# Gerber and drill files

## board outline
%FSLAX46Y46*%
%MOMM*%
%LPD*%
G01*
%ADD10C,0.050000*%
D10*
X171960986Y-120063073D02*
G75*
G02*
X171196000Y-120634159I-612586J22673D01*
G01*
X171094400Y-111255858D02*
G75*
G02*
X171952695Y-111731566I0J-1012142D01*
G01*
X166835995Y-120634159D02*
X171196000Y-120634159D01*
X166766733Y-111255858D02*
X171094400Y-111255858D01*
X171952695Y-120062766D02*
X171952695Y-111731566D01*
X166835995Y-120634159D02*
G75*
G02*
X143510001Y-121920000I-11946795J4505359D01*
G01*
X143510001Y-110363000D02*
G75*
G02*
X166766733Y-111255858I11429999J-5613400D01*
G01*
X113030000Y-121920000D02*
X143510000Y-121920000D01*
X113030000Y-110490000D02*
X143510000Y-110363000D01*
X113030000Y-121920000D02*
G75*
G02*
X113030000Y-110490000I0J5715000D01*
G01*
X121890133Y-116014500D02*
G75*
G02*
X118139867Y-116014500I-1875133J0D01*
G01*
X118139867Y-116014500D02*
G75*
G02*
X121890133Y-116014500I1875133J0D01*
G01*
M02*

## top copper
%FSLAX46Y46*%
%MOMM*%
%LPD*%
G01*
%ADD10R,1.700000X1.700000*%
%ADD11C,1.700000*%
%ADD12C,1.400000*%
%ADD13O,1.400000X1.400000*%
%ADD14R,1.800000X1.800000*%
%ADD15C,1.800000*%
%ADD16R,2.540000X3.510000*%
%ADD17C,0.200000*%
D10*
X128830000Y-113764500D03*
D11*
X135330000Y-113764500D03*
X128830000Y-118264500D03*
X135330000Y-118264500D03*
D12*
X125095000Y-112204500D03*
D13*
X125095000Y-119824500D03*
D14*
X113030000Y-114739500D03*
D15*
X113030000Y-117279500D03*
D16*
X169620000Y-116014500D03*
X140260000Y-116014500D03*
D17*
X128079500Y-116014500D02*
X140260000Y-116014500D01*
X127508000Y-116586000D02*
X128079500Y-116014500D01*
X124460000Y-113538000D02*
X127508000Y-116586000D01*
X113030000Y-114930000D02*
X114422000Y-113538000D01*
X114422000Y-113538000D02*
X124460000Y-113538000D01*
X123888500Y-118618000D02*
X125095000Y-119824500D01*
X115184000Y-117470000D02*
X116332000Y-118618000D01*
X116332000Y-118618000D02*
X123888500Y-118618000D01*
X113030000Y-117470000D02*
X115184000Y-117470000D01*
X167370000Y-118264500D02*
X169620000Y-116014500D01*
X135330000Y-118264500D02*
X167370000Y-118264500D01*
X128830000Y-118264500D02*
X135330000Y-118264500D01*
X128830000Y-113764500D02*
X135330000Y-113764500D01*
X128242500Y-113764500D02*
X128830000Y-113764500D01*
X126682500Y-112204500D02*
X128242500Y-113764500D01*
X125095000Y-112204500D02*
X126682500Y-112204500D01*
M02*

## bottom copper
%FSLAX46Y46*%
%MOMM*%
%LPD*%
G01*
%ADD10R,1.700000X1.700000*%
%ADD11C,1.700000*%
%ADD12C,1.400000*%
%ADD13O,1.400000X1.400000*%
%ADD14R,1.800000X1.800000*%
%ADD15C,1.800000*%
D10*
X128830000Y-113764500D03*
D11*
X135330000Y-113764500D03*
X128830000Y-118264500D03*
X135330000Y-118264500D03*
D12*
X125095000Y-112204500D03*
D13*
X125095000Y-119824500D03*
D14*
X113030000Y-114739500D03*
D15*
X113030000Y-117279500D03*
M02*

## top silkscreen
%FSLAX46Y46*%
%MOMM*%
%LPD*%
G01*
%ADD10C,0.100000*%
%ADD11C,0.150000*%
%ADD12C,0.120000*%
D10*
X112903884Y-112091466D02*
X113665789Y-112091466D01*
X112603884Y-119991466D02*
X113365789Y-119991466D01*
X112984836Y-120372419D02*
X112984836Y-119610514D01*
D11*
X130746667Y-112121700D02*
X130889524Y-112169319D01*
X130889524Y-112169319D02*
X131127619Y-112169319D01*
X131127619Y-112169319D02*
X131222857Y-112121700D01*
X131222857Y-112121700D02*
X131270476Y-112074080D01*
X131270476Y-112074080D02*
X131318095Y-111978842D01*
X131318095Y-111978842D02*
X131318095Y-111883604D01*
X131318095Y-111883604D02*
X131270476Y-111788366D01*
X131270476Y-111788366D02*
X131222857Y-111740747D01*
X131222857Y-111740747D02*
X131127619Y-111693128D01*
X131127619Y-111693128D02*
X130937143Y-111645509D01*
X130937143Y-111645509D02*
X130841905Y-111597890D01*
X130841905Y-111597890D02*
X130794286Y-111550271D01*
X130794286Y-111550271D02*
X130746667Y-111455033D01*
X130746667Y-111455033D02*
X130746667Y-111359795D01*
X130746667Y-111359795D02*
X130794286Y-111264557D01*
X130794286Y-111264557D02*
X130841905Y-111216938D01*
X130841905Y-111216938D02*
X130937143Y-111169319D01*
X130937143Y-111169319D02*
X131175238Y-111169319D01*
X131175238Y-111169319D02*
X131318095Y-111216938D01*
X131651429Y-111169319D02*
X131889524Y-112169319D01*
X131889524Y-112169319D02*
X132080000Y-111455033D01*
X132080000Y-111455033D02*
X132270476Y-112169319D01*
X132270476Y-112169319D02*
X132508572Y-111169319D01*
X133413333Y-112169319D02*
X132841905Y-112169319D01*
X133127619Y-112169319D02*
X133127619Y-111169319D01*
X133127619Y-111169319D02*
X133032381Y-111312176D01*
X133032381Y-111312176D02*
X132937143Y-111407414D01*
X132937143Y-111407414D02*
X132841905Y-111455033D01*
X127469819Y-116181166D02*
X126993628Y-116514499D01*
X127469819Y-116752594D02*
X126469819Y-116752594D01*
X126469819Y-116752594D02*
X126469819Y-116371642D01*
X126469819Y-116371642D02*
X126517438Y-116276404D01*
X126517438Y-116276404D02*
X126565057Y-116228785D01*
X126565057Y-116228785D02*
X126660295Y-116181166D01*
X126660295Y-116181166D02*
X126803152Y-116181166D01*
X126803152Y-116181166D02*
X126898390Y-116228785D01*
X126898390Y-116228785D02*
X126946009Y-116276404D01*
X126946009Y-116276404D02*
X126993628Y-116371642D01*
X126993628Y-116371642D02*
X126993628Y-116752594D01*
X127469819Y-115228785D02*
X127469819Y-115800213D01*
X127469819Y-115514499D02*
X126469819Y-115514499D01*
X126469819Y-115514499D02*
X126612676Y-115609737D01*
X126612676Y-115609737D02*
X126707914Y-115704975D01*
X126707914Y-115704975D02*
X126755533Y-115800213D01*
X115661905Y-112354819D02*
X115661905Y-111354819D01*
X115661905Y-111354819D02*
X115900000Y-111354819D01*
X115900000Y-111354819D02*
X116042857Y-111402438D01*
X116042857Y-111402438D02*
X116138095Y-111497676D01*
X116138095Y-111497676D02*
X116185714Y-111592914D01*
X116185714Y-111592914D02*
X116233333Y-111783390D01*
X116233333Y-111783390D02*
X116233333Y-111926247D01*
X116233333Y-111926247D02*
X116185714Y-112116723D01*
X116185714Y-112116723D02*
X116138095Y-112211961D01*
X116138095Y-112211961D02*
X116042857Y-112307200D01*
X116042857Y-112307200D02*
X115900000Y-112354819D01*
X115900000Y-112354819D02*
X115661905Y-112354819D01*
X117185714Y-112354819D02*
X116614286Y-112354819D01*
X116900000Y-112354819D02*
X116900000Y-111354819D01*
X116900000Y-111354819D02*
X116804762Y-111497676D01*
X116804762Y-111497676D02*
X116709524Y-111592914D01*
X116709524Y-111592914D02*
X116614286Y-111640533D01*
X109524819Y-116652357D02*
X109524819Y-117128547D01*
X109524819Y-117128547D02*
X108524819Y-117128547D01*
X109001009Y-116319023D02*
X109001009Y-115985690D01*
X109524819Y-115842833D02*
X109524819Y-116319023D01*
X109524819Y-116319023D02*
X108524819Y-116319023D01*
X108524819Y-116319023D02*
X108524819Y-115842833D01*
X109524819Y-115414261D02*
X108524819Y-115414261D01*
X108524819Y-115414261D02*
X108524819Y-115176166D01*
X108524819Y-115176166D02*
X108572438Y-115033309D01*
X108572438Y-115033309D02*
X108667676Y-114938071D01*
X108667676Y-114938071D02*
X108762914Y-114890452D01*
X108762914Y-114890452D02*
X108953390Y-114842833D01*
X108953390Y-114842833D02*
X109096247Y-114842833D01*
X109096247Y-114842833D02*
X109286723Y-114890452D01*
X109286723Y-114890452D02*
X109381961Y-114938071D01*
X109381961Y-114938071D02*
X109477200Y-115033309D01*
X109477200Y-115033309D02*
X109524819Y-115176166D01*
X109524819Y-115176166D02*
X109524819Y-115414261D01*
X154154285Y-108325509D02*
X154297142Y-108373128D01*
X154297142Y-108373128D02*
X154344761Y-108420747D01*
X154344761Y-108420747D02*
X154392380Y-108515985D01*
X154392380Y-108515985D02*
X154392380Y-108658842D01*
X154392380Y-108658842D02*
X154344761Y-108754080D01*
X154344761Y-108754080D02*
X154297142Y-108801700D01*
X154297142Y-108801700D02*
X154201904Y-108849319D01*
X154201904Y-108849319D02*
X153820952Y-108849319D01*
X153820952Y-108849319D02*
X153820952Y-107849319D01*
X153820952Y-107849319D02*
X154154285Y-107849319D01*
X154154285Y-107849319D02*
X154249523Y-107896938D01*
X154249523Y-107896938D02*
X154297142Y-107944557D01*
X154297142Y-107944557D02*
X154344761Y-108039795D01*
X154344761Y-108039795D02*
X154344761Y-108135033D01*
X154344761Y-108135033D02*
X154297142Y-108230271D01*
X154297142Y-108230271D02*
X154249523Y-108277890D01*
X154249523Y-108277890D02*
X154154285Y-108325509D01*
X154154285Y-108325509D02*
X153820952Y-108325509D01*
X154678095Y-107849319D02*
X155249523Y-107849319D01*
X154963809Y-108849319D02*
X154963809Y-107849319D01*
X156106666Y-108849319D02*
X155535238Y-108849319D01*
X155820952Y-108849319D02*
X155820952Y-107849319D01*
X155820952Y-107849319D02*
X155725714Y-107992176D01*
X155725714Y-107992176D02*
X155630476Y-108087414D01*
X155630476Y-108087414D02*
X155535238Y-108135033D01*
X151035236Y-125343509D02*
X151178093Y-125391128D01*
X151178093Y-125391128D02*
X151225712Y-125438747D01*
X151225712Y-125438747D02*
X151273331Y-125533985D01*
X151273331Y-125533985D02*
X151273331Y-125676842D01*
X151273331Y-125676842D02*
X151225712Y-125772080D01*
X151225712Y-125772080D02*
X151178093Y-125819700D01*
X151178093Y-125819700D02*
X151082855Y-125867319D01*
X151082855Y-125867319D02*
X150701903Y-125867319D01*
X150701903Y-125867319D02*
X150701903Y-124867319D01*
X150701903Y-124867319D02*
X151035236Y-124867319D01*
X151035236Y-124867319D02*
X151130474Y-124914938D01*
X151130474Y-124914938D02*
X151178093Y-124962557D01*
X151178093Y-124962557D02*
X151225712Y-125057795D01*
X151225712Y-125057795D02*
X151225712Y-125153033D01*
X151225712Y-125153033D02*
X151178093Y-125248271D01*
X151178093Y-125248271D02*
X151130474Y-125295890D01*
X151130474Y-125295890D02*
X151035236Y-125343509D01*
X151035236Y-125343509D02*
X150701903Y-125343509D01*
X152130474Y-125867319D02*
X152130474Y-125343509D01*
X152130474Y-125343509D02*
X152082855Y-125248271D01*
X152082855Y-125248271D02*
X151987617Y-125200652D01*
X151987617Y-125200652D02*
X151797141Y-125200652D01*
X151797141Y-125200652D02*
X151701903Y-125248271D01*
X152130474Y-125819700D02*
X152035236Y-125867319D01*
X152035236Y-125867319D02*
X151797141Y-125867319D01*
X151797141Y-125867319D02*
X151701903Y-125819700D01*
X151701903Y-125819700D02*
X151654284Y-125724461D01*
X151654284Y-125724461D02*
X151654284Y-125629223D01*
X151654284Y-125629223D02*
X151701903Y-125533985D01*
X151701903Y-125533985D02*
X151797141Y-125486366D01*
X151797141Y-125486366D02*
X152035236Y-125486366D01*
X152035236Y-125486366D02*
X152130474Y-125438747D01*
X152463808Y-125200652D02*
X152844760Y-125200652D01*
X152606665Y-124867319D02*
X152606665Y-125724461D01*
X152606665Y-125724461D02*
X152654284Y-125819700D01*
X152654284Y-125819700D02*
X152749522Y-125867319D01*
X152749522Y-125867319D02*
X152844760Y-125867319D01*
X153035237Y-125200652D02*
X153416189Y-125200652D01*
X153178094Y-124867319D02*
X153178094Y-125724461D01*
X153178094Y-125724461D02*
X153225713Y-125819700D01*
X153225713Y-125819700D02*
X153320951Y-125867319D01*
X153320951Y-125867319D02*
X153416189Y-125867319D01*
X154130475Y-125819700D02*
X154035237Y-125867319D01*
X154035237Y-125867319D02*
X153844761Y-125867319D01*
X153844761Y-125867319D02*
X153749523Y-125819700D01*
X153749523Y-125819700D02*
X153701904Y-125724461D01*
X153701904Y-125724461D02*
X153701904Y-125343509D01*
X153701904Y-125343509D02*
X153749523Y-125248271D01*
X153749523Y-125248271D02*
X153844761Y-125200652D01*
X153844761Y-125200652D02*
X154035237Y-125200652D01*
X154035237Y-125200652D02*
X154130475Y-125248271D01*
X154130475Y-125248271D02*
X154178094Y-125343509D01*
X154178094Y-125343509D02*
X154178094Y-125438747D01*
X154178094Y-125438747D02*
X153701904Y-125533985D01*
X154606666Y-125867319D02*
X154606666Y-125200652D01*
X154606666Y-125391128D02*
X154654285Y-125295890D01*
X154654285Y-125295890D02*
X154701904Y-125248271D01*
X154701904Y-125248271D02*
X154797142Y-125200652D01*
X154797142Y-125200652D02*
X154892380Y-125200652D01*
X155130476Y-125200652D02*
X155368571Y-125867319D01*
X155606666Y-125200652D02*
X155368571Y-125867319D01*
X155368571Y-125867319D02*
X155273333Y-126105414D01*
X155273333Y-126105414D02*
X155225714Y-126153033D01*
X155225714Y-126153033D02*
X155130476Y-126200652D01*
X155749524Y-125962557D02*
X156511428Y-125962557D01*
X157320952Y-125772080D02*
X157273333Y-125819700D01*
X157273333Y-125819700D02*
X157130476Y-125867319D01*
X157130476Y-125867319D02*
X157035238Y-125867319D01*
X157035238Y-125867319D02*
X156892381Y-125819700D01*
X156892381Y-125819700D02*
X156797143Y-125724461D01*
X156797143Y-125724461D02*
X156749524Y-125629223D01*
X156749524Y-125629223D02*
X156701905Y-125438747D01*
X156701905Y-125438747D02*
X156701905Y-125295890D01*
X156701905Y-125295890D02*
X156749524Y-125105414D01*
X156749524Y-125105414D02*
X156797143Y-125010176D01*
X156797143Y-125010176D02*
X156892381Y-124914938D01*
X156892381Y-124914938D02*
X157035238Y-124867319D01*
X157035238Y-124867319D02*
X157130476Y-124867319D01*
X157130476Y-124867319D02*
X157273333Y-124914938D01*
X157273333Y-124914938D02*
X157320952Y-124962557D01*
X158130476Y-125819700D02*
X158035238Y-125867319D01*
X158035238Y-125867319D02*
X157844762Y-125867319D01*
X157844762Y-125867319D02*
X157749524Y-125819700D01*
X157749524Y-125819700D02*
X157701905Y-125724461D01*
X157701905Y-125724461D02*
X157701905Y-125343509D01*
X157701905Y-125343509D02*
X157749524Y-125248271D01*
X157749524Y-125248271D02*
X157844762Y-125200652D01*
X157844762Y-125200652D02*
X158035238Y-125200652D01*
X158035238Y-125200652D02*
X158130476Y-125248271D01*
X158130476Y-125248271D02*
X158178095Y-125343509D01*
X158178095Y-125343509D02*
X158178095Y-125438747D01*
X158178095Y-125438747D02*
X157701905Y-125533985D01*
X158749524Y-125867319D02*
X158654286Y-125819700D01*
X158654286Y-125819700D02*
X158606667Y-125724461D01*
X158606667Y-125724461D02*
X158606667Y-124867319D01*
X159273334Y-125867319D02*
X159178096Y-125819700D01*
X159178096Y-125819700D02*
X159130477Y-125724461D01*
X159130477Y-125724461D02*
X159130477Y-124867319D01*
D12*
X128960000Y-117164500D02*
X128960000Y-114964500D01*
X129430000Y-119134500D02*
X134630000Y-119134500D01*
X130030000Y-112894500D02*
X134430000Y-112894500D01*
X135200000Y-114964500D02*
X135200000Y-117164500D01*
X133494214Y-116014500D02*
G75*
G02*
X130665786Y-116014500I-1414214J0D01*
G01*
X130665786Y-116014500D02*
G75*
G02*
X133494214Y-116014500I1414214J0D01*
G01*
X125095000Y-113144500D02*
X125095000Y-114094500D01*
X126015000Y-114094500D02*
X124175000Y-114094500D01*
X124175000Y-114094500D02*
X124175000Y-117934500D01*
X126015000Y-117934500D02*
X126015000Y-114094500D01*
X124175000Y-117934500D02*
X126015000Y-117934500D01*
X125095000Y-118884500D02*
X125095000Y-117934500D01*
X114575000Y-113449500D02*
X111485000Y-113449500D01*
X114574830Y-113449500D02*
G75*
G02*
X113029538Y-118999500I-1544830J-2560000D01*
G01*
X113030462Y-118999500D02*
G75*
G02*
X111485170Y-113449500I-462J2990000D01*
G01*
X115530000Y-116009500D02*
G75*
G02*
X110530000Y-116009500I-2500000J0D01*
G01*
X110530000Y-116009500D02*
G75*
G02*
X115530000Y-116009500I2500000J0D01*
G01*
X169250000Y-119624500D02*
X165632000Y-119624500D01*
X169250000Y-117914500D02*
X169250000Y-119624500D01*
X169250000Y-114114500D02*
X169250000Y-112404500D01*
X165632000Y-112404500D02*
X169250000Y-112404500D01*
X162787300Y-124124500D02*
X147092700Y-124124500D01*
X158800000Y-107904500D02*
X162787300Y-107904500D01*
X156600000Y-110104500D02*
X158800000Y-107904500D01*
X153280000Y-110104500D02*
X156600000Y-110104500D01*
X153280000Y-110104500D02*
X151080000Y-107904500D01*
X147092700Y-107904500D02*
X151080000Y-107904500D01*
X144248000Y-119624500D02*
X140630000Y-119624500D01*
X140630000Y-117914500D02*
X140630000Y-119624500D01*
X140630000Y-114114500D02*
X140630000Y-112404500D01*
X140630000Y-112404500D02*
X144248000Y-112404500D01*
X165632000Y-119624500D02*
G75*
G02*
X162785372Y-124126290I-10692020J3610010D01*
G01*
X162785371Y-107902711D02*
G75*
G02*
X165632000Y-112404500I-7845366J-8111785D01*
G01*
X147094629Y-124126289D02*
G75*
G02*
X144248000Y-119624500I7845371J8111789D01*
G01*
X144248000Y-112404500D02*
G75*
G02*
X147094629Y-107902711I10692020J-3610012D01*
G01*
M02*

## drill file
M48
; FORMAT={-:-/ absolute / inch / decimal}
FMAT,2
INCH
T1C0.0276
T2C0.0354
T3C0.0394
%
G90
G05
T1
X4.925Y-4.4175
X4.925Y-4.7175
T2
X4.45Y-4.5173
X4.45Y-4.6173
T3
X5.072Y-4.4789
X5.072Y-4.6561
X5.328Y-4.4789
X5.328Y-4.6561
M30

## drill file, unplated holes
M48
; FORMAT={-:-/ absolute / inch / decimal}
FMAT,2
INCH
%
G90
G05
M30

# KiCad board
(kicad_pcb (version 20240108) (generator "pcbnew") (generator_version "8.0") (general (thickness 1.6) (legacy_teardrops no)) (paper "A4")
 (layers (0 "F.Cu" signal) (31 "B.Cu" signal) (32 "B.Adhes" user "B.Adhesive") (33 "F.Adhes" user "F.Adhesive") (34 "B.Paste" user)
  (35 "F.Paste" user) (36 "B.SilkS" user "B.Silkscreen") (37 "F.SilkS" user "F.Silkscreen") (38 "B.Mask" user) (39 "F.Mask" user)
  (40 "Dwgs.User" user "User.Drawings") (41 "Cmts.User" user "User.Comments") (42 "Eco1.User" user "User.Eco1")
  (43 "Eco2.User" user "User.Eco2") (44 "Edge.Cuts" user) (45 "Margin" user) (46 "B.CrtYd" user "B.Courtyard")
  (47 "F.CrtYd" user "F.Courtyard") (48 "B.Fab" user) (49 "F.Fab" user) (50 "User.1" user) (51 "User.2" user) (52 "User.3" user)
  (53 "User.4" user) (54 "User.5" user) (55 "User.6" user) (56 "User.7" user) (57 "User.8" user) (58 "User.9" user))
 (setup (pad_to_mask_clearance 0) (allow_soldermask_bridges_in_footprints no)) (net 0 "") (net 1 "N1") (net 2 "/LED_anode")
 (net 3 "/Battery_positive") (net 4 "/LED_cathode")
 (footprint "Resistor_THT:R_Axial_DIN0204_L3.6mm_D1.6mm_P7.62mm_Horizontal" (layer "F.Cu") (at 125.095 112.2045 -90)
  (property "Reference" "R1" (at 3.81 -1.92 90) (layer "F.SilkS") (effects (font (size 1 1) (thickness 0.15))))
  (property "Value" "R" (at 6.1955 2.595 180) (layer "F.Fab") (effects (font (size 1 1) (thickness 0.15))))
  (fp_line (start 1.89 0.92) (end 5.73 0.92) (stroke (width 0.12) (type solid)) (layer "F.SilkS"))
  (fp_line (start 5.73 0.92) (end 5.73 -0.92) (stroke (width 0.12) (type solid)) (layer "F.SilkS"))
  (fp_line (start 0.94 0) (end 1.89 0) (stroke (width 0.12) (type solid)) (layer "F.SilkS"))
  (fp_line (start 6.68 0) (end 5.73 0) (stroke (width 0.12) (type solid)) (layer "F.SilkS"))
  (fp_line (start 1.89 -0.92) (end 1.89 0.92) (stroke (width 0.12) (type solid)) (layer "F.SilkS"))
  (fp_line (start 5.73 -0.92) (end 1.89 -0.92) (stroke (width 0.12) (type solid)) (layer "F.SilkS"))
  (pad "1" thru_hole circle (at 0 0 270) (size 1.4 1.4) (drill 0.7) (layers "*.Cu" "*.Mask") (remove_unused_layers no) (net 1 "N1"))
  (pad "2" thru_hole oval (at 7.62 0 270) (size 1.4 1.4) (drill 0.7) (layers "*.Cu" "*.Mask") (remove_unused_layers no) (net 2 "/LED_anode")))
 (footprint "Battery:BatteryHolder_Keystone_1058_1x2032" (layer "F.Cu") (at 154.94 116.0145 180)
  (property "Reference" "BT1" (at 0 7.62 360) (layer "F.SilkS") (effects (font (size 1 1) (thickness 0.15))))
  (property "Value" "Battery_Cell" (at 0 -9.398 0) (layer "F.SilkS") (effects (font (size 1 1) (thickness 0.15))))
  (fp_line (start 14.31 3.61) (end 10.692 3.61) (stroke (width 0.12) (type solid)) (layer "F.SilkS"))
  (fp_line (start 14.31 1.9) (end 14.31 3.61) (stroke (width 0.12) (type solid)) (layer "F.SilkS"))
  (fp_line (start 14.31 -1.9) (end 14.31 -3.61) (stroke (width 0.12) (type solid)) (layer "F.SilkS"))
  (fp_line (start 10.692 -3.61) (end 14.31 -3.61) (stroke (width 0.12) (type solid)) (layer "F.SilkS"))
  (fp_line (start 7.8473 8.11) (end 3.86 8.11) (stroke (width 0.12) (type solid)) (layer "F.SilkS"))
  (fp_line (start 1.66 5.91) (end 3.86 8.11) (stroke (width 0.12) (type solid)) (layer "F.SilkS"))
  (fp_line (start 1.66 5.91) (end -1.66 5.91) (stroke (width 0.12) (type solid)) (layer "F.SilkS"))
  (fp_line (start -1.66 5.91) (end -3.86 8.11) (stroke (width 0.12) (type solid)) (layer "F.SilkS"))
  (fp_line (start -3.86 8.11) (end -7.8473 8.11) (stroke (width 0.12) (type solid)) (layer "F.SilkS"))
  (fp_line (start -7.8473 -8.11) (end 7.8473 -8.11) (stroke (width 0.12) (type solid)) (layer "F.SilkS"))
  (fp_line (start -10.692 3.61) (end -14.31 3.61) (stroke (width 0.12) (type solid)) (layer "F.SilkS"))
  (fp_line (start -14.31 1.9) (end -14.31 3.61) (stroke (width 0.12) (type solid)) (layer "F.SilkS"))
  (fp_line (start -14.31 -1.9) (end -14.31 -3.61) (stroke (width 0.12) (type solid)) (layer "F.SilkS"))
  (fp_line (start -14.31 -3.61) (end -10.692 -3.61) (stroke (width 0.12) (type solid)) (layer "F.SilkS"))
  (fp_arc (start 10.692 3.61) (mid 9.538084 6.031244) (end 7.845371 8.111789) (stroke (width 0.12) (type solid)) (layer "F.SilkS"))
  (fp_arc (start 7.845371 -8.111789) (mid 9.538085 -6.031244) (end 10.692 -3.61) (stroke (width 0.12) (type solid)) (layer "F.SilkS"))
  (fp_arc (start -7.845371 8.111789) (mid -9.538085 6.031244) (end -10.692 3.61) (stroke (width 0.12) (type solid)) (layer "F.SilkS"))
  (fp_arc (start -10.692 -3.61) (mid -9.538084 -6.031244) (end -7.845371 -8.111789) (stroke (width 0.12) (type solid)) (layer "F.SilkS"))
  (pad "1" smd rect (at -14.68 0 180) (size 2.54 3.51) (layers "F.Cu" "F.Paste" "F.Mask") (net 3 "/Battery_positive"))
  (pad "2" smd rect (at 14.68 0 180) (size 2.54 3.51) (layers "F.Cu" "F.Paste" "F.Mask") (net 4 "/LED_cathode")))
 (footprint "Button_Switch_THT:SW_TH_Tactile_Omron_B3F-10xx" (layer "F.Cu") (at 128.83 113.7645)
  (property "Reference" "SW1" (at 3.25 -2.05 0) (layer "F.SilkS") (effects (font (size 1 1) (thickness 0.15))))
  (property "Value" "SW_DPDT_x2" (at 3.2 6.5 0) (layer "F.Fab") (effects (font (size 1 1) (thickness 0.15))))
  (fp_line (start 0.13 3.4) (end 0.13 1.2) (stroke (width 0.12) (type solid)) (layer "F.SilkS"))
  (fp_line (start 0.6 5.37) (end 5.8 5.37) (stroke (width 0.12) (type solid)) (layer "F.SilkS"))
  (fp_line (start 1.2 -0.87) (end 5.6 -0.87) (stroke (width 0.12) (type solid)) (layer "F.SilkS"))
  (fp_line (start 6.37 1.2) (end 6.37 3.4) (stroke (width 0.12) (type solid)) (layer "F.SilkS"))
  (fp_circle (center 3.25 2.25) (end 4.25 3.25) (stroke (width 0.12) (type solid)) (fill none) (layer "F.SilkS"))
  (pad "1" thru_hole rect (at 0 0) (size 1.7 1.7) (drill 1) (layers "*.Cu" "*.Mask") (remove_unused_layers no) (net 1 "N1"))
  (pad "1" thru_hole circle (at 6.5 0) (size 1.7 1.7) (drill 1) (layers "*.Cu" "*.Mask") (remove_unused_layers no) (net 1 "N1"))
  (pad "2" thru_hole circle (at 0 4.5) (size 1.7 1.7) (drill 1) (layers "*.Cu" "*.Mask") (remove_unused_layers no)
   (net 3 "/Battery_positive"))
  (pad "2" thru_hole circle (at 6.5 4.5) (size 1.7 1.7) (drill 1) (layers "*.Cu" "*.Mask") (remove_unused_layers no)
   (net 3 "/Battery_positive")))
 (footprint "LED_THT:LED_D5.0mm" (layer "F.Cu") (at 113.03 114.7395 -90)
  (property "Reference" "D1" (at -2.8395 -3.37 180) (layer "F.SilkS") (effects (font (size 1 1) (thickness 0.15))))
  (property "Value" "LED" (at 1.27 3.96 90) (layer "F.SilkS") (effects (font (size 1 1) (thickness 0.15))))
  (fp_line (start -1.29 -1.545) (end -1.29 1.545) (stroke (width 0.12) (type solid)) (layer "F.SilkS"))
  (fp_arc (start 4.26 -0.000462) (mid 2.072002 2.880433) (end -1.29 1.54483) (stroke (width 0.12) (type solid)) (layer "F.SilkS"))
  (fp_arc (start -1.29 -1.54483) (mid 2.072002 -2.880433) (end 4.26 0.000462) (stroke (width 0.12) (type solid)) (layer "F.SilkS"))
  (fp_circle (center 1.27 0) (end 3.77 0) (stroke (width 0.12) (type solid)) (fill none) (layer "F.SilkS"))
  (pad "1" thru_hole rect (at 0 0 270) (size 1.8 1.8) (drill 0.9) (layers "*.Cu" "*.Mask") (remove_unused_layers no) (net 4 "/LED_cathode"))
  (pad "2" thru_hole circle (at 2.54 0 270) (size 1.8 1.8) (drill 0.9) (layers "*.Cu" "*.Mask") (remove_unused_layers no)
   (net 2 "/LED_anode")))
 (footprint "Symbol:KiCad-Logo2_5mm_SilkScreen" (layer "B.Cu") (at 154.178 113.03 180)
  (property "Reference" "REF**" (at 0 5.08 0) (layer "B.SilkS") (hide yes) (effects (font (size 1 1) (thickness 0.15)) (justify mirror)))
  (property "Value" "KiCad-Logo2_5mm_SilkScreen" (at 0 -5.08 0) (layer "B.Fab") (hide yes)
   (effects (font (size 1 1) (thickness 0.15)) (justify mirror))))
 (gr_line (start 113.03 121.92) (end 143.51 121.92) (locked yes) (stroke (width 0.05) (type default)) (layer "Edge.Cuts"))
 (gr_line (start 166.835995 120.634159) (end 171.196 120.634159) (locked yes) (stroke (width 0.05) (type default)) (layer "Edge.Cuts"))
 (gr_arc (start 143.510001 110.363) (mid 155.428516 103.251759) (end 166.766733 111.255858) (locked yes)
  (stroke (width 0.05) (type default)) (layer "Edge.Cuts"))
 (gr_line (start 171.952695 120.062766) (end 171.952695 111.731566) (locked yes) (stroke (width 0.05) (type default)) (layer "Edge.Cuts"))
 (gr_arc (start 171.960986 120.063073) (mid 171.715112 120.531621) (end 171.196 120.634159) (locked yes)
  (stroke (width 0.05) (type default)) (layer "Edge.Cuts"))
 (gr_arc (start 171.0944 111.255858) (mid 171.585055 111.382738) (end 171.952695 111.731566) (locked yes)
  (stroke (width 0.05) (type default)) (layer "Edge.Cuts"))
 (gr_arc (start 166.835995 120.634159) (mid 155.591972 128.877537) (end 143.510001 121.92) (locked yes) (stroke (width 0.05) (type default))
  (layer "Edge.Cuts"))
 (gr_line (start 166.766733 111.255858) (end 171.0944 111.255858) (locked yes) (stroke (width 0.05) (type default)) (layer "Edge.Cuts"))
 (gr_arc (start 113.03 121.92) (mid 107.315 116.205) (end 113.03 110.49) (locked yes) (stroke (width 0.05) (type default))
  (layer "Edge.Cuts"))
 (gr_line (start 113.03 110.49) (end 143.51 110.363) (locked yes) (stroke (width 0.05) (type default)) (layer "Edge.Cuts"))
 (gr_circle (center 120.015 116.0145) (end 120.904 114.3635) (stroke (width 0.05) (type default)) (fill none) (layer "Edge.Cuts"))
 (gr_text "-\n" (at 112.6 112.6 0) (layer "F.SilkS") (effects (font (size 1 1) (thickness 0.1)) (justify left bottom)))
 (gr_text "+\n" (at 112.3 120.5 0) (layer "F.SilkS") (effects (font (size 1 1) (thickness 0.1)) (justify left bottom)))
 (segment (start 127.508 116.586) (end 128.0795 116.0145) (width 0.2) (layer "F.Cu") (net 4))
 (segment (start 128.0795 116.0145) (end 140.26 116.0145) (width 0.2) (layer "F.Cu") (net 4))
 (segment (start 114.422 113.538) (end 124.46 113.538) (width 0.2) (layer "F.Cu") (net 4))
 (segment (start 124.46 113.538) (end 127.508 116.586) (width 0.2) (layer "F.Cu") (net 4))
 (segment (start 113.03 114.93) (end 114.422 113.538) (width 0.2) (layer "F.Cu") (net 4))
 (segment (start 135.33 118.2645) (end 167.37 118.2645) (width 0.2) (layer "F.Cu") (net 3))
 (segment (start 167.37 118.2645) (end 169.62 116.0145) (width 0.2) (layer "F.Cu") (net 3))
 (segment (start 128.83 118.2645) (end 135.33 118.2645) (width 0.2) (layer "F.Cu") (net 3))
 (segment (start 113.03 117.47) (end 115.184 117.47) (width 0.2) (layer "F.Cu") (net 2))
 (segment (start 116.332 118.618) (end 123.8885 118.618) (width 0.2) (layer "F.Cu") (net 2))
 (segment (start 115.184 117.47) (end 116.332 118.618) (width 0.2) (layer "F.Cu") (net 2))
 (segment (start 123.8885 118.618) (end 125.095 119.8245) (width 0.2) (layer "F.Cu") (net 2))
 (segment (start 128.83 113.7645) (end 135.33 113.7645) (width 0.2) (layer "F.Cu") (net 1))
 (segment (start 126.6825 112.2045) (end 128.2425 113.7645) (width 0.2) (layer "F.Cu") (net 1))
 (segment (start 125.095 112.2045) (end 126.6825 112.2045) (width 0.2) (layer "F.Cu") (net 1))
 (segment (start 128.2425 113.7645) (end 128.83 113.7645) (width 0.2) (layer "F.Cu") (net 1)))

